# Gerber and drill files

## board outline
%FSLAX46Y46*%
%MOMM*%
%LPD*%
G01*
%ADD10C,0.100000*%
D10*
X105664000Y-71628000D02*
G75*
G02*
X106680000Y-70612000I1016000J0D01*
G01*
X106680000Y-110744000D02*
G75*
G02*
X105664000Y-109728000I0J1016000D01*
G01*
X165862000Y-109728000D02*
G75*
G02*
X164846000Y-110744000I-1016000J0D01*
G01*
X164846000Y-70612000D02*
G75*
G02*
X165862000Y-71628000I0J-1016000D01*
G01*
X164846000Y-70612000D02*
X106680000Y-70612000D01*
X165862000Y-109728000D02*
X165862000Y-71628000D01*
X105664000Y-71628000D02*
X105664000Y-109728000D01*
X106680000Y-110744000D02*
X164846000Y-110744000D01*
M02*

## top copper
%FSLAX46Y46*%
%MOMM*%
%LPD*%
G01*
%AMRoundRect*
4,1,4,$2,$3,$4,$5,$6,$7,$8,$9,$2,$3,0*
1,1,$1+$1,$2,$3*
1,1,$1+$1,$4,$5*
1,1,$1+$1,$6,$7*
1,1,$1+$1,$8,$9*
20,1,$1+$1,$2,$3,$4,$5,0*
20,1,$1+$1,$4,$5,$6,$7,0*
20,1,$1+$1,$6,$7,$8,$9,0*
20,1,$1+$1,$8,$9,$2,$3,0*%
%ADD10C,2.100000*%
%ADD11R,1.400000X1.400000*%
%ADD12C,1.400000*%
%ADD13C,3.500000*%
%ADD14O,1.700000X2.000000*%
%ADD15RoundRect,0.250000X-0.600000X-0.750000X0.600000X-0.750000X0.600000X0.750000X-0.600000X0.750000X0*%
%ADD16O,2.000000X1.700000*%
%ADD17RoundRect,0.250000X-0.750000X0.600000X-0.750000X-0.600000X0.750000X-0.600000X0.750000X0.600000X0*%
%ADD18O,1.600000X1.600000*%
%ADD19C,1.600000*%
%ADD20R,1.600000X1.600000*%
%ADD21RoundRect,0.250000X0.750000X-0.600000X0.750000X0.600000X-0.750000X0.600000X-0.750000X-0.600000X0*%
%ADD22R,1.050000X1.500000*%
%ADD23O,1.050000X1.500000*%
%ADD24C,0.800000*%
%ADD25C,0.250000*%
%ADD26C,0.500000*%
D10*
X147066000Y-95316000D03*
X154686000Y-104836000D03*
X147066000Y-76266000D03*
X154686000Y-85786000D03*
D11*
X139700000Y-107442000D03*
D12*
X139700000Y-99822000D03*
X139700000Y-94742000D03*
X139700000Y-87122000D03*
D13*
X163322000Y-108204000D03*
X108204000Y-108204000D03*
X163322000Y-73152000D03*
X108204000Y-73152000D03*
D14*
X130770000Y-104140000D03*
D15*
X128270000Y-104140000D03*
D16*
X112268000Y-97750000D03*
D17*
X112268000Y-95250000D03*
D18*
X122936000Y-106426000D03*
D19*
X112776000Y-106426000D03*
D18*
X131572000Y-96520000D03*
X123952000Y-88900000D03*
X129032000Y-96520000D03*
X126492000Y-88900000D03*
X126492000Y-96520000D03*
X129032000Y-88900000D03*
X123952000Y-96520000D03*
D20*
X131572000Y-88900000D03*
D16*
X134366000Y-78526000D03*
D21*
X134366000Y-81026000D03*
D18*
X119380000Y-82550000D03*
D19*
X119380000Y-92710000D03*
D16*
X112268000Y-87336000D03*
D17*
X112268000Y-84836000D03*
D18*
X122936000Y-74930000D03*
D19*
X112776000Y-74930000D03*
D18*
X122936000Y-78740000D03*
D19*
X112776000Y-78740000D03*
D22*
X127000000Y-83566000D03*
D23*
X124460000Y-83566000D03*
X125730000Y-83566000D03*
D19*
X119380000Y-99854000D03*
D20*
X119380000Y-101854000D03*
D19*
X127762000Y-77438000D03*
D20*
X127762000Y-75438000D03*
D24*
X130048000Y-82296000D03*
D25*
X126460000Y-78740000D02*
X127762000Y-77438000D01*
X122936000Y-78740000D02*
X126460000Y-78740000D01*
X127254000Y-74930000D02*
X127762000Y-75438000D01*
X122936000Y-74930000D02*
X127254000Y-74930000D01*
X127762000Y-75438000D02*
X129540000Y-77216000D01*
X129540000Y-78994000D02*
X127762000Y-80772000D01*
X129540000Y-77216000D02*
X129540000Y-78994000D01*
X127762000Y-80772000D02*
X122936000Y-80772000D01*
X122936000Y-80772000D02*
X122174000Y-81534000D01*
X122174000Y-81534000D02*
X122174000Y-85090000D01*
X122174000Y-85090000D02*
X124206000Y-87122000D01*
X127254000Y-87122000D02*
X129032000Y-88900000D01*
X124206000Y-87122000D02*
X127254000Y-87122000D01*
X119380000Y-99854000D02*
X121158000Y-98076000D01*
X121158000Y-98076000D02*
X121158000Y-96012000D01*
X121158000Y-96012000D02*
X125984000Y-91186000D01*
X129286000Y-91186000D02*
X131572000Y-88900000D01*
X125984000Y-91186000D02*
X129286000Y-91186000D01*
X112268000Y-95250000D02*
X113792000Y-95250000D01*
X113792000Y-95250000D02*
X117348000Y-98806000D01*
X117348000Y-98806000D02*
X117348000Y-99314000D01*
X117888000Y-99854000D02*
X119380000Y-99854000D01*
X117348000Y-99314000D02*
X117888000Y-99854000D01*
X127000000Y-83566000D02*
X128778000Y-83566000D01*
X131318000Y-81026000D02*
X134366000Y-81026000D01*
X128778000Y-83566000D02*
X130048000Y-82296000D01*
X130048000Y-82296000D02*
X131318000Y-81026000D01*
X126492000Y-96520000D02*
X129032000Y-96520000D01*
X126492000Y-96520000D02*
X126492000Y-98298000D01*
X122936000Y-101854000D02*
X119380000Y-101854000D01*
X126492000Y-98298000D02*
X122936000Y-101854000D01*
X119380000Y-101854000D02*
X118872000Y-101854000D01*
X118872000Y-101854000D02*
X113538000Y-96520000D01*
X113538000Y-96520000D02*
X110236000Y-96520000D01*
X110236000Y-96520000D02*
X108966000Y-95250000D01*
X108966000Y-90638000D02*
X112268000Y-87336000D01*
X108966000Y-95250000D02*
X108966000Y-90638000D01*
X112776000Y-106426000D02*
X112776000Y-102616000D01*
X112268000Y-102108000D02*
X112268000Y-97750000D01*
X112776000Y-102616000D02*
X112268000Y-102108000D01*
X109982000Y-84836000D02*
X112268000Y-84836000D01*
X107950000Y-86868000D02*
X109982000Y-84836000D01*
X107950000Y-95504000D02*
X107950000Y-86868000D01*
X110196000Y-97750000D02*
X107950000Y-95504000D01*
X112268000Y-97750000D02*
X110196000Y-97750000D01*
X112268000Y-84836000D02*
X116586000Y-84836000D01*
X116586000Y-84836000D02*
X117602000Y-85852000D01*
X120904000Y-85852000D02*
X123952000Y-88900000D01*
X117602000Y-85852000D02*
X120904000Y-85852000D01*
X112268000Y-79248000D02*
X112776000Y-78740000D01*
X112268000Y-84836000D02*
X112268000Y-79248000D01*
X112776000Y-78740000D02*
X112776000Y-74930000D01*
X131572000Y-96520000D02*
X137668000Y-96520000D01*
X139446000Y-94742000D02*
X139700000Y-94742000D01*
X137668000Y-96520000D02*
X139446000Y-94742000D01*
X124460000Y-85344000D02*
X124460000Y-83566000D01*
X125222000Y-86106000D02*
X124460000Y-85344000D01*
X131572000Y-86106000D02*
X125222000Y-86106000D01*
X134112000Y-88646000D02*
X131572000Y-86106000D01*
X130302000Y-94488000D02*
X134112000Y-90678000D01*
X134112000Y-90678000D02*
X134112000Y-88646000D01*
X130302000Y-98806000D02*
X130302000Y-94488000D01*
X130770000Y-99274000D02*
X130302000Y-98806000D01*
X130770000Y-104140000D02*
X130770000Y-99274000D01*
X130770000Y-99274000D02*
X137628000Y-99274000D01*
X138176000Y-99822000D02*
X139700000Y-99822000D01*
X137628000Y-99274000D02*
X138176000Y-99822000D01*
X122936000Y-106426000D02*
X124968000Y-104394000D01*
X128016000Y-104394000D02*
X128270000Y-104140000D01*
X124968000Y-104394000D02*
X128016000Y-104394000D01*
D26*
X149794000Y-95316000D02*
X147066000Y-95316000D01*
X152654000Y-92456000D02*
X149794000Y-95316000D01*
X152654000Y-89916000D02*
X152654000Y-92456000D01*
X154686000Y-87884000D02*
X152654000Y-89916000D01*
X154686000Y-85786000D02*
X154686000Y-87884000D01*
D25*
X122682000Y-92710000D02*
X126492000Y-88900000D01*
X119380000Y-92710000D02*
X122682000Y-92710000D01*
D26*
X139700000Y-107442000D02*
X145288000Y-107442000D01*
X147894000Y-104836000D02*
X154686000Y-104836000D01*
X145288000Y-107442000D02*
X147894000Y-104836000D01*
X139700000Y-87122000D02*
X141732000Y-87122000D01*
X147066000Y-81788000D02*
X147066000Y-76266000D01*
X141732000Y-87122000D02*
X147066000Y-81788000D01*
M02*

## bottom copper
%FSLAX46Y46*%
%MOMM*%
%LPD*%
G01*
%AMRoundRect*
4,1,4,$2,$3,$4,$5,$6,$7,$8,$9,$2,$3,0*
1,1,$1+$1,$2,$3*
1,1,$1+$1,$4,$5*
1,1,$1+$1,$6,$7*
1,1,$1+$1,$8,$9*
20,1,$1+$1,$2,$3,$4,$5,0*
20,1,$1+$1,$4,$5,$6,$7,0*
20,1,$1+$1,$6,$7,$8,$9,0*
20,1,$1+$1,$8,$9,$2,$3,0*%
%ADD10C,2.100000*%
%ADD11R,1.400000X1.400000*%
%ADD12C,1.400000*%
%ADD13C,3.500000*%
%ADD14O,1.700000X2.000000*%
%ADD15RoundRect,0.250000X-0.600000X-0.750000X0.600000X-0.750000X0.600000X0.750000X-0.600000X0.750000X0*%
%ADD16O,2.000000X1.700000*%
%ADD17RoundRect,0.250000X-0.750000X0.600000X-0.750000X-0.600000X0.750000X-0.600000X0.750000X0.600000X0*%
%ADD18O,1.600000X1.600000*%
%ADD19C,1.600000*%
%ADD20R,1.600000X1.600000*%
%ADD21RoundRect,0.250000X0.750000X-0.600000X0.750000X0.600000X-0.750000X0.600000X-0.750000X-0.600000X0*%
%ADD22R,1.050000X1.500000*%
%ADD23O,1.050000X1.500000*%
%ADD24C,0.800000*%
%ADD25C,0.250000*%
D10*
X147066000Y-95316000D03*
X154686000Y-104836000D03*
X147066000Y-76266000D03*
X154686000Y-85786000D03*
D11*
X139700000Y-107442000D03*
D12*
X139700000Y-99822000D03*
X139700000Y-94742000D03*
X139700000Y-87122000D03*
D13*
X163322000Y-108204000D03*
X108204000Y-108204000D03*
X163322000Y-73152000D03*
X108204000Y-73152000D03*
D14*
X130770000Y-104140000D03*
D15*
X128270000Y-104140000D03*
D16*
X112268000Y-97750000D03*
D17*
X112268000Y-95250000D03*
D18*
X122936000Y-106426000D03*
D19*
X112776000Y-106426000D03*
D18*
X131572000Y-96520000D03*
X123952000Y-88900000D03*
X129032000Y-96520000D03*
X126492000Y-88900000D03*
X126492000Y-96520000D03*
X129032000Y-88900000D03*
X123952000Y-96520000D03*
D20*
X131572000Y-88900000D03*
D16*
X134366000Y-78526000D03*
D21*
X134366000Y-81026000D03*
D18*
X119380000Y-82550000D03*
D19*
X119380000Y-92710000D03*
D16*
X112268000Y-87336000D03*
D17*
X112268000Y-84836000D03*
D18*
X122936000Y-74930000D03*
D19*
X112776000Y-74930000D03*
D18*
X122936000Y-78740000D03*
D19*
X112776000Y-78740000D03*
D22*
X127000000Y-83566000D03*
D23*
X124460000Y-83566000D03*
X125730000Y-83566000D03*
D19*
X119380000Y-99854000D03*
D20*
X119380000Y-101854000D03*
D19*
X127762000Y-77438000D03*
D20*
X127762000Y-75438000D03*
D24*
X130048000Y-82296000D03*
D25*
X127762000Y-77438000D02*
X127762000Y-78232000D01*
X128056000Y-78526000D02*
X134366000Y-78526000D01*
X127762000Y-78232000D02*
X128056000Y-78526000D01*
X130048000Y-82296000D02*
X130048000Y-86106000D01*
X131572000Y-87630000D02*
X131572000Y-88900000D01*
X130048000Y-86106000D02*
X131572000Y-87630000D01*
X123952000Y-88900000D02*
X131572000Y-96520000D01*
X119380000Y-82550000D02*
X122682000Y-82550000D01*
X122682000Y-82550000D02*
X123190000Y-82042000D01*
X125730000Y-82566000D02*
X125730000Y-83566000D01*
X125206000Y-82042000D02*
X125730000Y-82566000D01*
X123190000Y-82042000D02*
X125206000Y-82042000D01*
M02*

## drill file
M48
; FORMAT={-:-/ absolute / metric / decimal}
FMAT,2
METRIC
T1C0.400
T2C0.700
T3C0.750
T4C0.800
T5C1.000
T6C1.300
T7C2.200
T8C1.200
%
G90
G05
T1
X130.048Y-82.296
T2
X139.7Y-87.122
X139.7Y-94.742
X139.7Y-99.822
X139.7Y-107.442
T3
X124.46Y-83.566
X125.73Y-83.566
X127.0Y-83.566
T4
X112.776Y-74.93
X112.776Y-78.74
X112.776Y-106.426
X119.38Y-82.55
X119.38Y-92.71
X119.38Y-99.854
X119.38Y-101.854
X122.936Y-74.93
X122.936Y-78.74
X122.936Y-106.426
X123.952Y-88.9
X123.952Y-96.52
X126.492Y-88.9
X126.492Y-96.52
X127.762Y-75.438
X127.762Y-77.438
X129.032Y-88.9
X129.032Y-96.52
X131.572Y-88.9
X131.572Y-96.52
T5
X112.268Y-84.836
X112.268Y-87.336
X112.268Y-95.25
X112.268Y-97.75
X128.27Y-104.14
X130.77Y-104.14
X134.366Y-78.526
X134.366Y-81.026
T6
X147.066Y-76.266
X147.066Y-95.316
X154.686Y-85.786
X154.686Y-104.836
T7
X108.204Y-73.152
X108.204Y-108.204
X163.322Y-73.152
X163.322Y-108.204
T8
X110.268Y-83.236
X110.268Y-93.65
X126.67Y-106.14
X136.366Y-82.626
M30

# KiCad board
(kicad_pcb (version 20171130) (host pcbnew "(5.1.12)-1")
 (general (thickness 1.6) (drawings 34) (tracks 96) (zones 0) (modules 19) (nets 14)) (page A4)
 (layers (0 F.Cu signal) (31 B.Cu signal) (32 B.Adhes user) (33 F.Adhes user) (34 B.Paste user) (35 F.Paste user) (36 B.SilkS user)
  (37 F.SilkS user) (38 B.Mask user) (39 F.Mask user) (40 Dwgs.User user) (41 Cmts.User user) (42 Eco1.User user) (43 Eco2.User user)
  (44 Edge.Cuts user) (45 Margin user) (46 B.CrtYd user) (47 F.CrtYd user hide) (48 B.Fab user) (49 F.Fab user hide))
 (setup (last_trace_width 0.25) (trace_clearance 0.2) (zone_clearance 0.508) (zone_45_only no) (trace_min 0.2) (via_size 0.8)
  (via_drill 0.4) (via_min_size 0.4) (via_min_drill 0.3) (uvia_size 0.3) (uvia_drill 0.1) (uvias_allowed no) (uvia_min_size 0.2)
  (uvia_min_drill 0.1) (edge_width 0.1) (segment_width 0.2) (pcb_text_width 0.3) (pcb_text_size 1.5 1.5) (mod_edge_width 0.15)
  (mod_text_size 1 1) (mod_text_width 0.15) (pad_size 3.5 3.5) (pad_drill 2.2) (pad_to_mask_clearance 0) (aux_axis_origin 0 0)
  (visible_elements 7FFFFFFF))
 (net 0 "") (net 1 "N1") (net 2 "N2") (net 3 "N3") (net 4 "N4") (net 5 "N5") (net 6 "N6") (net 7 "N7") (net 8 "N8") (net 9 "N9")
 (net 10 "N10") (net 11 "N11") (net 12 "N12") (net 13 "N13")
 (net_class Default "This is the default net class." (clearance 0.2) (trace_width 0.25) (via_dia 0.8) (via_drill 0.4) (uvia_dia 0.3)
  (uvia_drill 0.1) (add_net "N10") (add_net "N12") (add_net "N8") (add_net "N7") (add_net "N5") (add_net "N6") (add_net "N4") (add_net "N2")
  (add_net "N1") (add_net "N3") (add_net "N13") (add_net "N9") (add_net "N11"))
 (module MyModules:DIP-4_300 (layer F.Cu) (at 150.876 100.076 90)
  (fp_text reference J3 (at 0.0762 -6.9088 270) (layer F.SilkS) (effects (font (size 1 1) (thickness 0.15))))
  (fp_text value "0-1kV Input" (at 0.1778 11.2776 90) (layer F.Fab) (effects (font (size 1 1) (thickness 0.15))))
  (pad 2 thru_hole circle (at 4.76 -3.81 90) (size 2.1 2.1) (drill 1.3) (layers *.Cu *.Mask) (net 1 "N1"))
  (pad 1 thru_hole circle (at -4.76 3.81 90) (size 2.1 2.1) (drill 1.3) (layers *.Cu *.Mask) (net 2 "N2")))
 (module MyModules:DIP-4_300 (layer F.Cu) (at 150.876 81.026 90)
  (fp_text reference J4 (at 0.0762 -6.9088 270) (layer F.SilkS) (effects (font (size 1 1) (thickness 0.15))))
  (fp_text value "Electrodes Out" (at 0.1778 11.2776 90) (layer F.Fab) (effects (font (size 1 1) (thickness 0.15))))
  (pad 2 thru_hole circle (at 4.76 -3.81 90) (size 2.1 2.1) (drill 1.3) (layers *.Cu *.Mask) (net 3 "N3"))
  (pad 1 thru_hole circle (at -4.76 3.81 90) (size 2.1 2.1) (drill 1.3) (layers *.Cu *.Mask) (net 1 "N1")))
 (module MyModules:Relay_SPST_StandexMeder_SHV (layer F.Cu) (at 139.7 107.442 90)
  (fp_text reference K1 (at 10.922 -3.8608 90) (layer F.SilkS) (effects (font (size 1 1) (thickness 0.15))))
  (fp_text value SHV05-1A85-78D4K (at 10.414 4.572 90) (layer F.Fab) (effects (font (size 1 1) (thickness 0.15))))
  (pad 1 thru_hole rect (at 0 0 90) (size 1.4 1.4) (drill 0.7) (layers *.Cu *.Mask) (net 2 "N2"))
  (pad 3 thru_hole circle (at 7.62 0 90) (size 1.4 1.4) (drill 0.7) (layers *.Cu *.Mask) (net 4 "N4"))
  (pad 5 thru_hole circle (at 12.7 0 90) (size 1.4 1.4) (drill 0.7) (layers *.Cu *.Mask) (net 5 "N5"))
  (pad 7 thru_hole circle (at 20.32 0 90) (size 1.4 1.4) (drill 0.7) (layers *.Cu *.Mask) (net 3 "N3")))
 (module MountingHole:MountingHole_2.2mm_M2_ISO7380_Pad (layer F.Cu) (at 163.322 108.204)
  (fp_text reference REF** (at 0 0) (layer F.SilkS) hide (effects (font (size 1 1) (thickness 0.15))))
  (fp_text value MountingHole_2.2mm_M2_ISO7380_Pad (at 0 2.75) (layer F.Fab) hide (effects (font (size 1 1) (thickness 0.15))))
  (pad 1 thru_hole circle (at 0 0) (size 3.5 3.5) (drill 2.2) (layers *.Cu *.Mask)))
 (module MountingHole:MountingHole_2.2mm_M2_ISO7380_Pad (layer F.Cu) (at 108.204 108.204)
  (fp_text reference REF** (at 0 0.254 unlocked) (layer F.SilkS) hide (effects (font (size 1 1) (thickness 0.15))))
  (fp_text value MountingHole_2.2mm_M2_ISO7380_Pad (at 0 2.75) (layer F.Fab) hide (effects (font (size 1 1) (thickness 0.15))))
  (pad 1 thru_hole circle (at 0 0) (size 3.5 3.5) (drill 2.2) (layers *.Cu *.Mask)))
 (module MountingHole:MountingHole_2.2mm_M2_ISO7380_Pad (layer F.Cu) (at 163.322 73.152)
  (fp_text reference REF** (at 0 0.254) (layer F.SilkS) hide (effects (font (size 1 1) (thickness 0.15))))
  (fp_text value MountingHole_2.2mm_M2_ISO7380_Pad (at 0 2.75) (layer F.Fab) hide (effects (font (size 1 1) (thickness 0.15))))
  (pad 1 thru_hole circle (at 0 0) (size 3.5 3.5) (drill 2.2) (layers *.Cu *.Mask)))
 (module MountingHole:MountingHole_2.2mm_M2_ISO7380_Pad (layer F.Cu) (at 108.204 73.152)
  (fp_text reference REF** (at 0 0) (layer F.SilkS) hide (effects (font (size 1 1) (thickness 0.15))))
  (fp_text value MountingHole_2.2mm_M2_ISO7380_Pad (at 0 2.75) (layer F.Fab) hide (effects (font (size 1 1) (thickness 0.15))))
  (pad 1 thru_hole circle (at 0 0) (size 3.5 3.5) (drill 2.2) (layers *.Cu *.Mask)))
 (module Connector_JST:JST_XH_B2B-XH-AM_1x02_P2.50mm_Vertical (layer F.Cu) (at 128.27 104.14)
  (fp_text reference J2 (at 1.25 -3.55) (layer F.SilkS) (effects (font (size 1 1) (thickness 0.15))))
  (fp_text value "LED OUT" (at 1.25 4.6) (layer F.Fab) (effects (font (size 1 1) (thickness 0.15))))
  (pad "" np_thru_hole circle (at -1.6 2) (size 1.2 1.2) (drill 1.2) (layers *.Cu *.Mask))
  (pad 2 thru_hole oval (at 2.5 0) (size 1.7 2) (drill 1) (layers *.Cu *.Mask) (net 4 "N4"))
  (pad 1 thru_hole roundrect (at 0 0) (size 1.7 2) (drill 1) (layers *.Cu *.Mask) (roundrect_rratio 0.147059) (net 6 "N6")))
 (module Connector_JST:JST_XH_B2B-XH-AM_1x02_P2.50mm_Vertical (layer F.Cu) (at 112.268 95.25 270)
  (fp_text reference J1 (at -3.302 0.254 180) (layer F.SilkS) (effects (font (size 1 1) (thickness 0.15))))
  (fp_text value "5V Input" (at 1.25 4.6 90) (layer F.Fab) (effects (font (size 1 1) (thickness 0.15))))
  (pad "" np_thru_hole circle (at -1.6 2 270) (size 1.2 1.2) (drill 1.2) (layers *.Cu *.Mask))
  (pad 2 thru_hole oval (at 2.5 0 270) (size 1.7 2) (drill 1) (layers *.Cu *.Mask) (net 5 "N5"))
  (pad 1 thru_hole roundrect (at 0 0 270) (size 1.7 2) (drill 1) (layers *.Cu *.Mask) (roundrect_rratio 0.147059) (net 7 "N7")))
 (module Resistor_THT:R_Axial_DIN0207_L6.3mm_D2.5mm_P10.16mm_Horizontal (layer F.Cu) (at 112.776 106.426)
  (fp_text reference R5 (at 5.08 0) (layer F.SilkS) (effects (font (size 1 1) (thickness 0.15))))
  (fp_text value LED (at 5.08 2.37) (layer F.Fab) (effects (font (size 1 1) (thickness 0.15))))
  (pad 2 thru_hole oval (at 10.16 0) (size 1.6 1.6) (drill 0.8) (layers *.Cu *.Mask) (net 6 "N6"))
  (pad 1 thru_hole circle (at 0 0) (size 1.6 1.6) (drill 0.8) (layers *.Cu *.Mask) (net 5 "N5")))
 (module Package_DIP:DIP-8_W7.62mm (layer F.Cu) (at 131.572 88.9 270)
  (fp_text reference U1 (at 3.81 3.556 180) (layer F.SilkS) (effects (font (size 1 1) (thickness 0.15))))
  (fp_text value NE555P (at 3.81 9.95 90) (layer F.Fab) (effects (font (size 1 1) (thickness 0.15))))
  (pad 8 thru_hole oval (at 7.62 0 270) (size 1.6 1.6) (drill 0.8) (layers *.Cu *.Mask) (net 5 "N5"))
  (pad 4 thru_hole oval (at 0 7.62 270) (size 1.6 1.6) (drill 0.8) (layers *.Cu *.Mask) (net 5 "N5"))
  (pad 7 thru_hole oval (at 7.62 2.54 270) (size 1.6 1.6) (drill 0.8) (layers *.Cu *.Mask) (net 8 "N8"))
  (pad 3 thru_hole oval (at 0 5.08 270) (size 1.6 1.6) (drill 0.8) (layers *.Cu *.Mask) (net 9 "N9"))
  (pad 6 thru_hole oval (at 7.62 5.08 270) (size 1.6 1.6) (drill 0.8) (layers *.Cu *.Mask) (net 8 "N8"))
  (pad 2 thru_hole oval (at 0 2.54 270) (size 1.6 1.6) (drill 0.8) (layers *.Cu *.Mask) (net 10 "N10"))
  (pad 5 thru_hole oval (at 7.62 7.62 270) (size 1.6 1.6) (drill 0.8) (layers *.Cu *.Mask) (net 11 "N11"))
  (pad 1 thru_hole rect (at 0 0 270) (size 1.6 1.6) (drill 0.8) (layers *.Cu *.Mask) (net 7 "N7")))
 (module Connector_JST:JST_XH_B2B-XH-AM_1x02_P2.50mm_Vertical (layer F.Cu) (at 134.366 81.026 90)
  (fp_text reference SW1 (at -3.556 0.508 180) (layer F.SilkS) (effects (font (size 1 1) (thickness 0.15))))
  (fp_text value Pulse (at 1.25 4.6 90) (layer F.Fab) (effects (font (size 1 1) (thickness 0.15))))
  (pad "" np_thru_hole circle (at -1.6 2 90) (size 1.2 1.2) (drill 1.2) (layers *.Cu *.Mask))
  (pad 2 thru_hole oval (at 2.5 0 90) (size 1.7 2) (drill 1) (layers *.Cu *.Mask) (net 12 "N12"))
  (pad 1 thru_hole roundrect (at 0 0 90) (size 1.7 2) (drill 1) (layers *.Cu *.Mask) (roundrect_rratio 0.147059) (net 7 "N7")))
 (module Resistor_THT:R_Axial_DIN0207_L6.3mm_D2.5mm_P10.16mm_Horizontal (layer F.Cu) (at 119.38 92.71 90)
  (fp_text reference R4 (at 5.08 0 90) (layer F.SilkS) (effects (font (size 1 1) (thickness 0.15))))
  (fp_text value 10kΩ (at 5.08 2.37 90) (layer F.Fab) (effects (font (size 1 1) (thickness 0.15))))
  (pad 2 thru_hole oval (at 10.16 0 90) (size 1.6 1.6) (drill 0.8) (layers *.Cu *.Mask) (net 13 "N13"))
  (pad 1 thru_hole circle (at 0 0 90) (size 1.6 1.6) (drill 0.8) (layers *.Cu *.Mask) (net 9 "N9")))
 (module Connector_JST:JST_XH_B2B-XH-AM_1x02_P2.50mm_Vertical (layer F.Cu) (at 112.268 84.836 270)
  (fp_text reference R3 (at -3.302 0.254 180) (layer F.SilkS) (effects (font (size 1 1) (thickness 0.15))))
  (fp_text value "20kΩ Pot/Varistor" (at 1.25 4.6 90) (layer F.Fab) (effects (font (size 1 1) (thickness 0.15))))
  (pad "" np_thru_hole circle (at -1.6 2 270) (size 1.2 1.2) (drill 1.2) (layers *.Cu *.Mask))
  (pad 2 thru_hole oval (at 2.5 0 270) (size 1.7 2) (drill 1) (layers *.Cu *.Mask) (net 8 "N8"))
  (pad 1 thru_hole roundrect (at 0 0 270) (size 1.7 2) (drill 1) (layers *.Cu *.Mask) (roundrect_rratio 0.147059) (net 5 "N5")))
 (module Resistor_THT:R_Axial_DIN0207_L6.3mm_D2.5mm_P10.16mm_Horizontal (layer F.Cu) (at 112.776 74.93)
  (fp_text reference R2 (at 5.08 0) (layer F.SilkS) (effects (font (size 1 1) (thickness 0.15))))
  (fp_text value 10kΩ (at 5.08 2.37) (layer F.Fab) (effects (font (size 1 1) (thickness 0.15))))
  (pad 2 thru_hole oval (at 10.16 0) (size 1.6 1.6) (drill 0.8) (layers *.Cu *.Mask) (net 10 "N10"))
  (pad 1 thru_hole circle (at 0 0) (size 1.6 1.6) (drill 0.8) (layers *.Cu *.Mask) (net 5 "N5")))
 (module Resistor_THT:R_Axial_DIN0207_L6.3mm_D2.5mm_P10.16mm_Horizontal (layer F.Cu) (at 112.776 78.74)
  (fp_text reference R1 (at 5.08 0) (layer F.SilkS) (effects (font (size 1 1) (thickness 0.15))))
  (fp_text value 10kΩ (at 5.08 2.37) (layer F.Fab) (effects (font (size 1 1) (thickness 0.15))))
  (pad 2 thru_hole oval (at 10.16 0) (size 1.6 1.6) (drill 0.8) (layers *.Cu *.Mask) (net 12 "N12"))
  (pad 1 thru_hole circle (at 0 0) (size 1.6 1.6) (drill 0.8) (layers *.Cu *.Mask) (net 5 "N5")))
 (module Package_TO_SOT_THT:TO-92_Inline (layer F.Cu) (at 127 83.566 180)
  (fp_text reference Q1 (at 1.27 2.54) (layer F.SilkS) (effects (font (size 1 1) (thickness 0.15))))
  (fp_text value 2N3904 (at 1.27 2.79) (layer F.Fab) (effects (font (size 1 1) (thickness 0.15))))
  (pad 1 thru_hole rect (at 0 0 180) (size 1.05 1.5) (drill 0.75) (layers *.Cu *.Mask) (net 7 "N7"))
  (pad 3 thru_hole oval (at 2.54 0 180) (size 1.05 1.5) (drill 0.75) (layers *.Cu *.Mask) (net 4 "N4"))
  (pad 2 thru_hole oval (at 1.27 0 180) (size 1.05 1.5) (drill 0.75) (layers *.Cu *.Mask) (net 13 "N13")))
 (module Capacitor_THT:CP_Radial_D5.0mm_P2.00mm (layer F.Cu) (at 119.38 101.854 90)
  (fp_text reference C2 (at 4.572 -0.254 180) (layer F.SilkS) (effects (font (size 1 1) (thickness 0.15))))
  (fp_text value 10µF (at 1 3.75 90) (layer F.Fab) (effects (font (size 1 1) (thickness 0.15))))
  (pad 2 thru_hole circle (at 2 0 90) (size 1.6 1.6) (drill 0.8) (layers *.Cu *.Mask) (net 7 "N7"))
  (pad 1 thru_hole rect (at 0 0 90) (size 1.6 1.6) (drill 0.8) (layers *.Cu *.Mask) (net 8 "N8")))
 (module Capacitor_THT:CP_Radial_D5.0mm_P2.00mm (layer F.Cu) (at 127.762 75.438 270)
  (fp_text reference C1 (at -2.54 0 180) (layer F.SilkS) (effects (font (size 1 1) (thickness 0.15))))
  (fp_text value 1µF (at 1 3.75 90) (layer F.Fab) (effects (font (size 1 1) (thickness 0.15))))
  (pad 2 thru_hole circle (at 2 0 270) (size 1.6 1.6) (drill 0.8) (layers *.Cu *.Mask) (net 12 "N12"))
  (pad 1 thru_hole rect (at 0 0 270) (size 1.6 1.6) (drill 0.8) (layers *.Cu *.Mask) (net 10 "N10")))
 (gr_arc (start 106.68 71.628) (end 106.68 70.612) (angle -90) (layer Edge.Cuts) (width 0.1))
 (gr_arc (start 106.68 109.728) (end 105.664 109.728) (angle -90) (layer Edge.Cuts) (width 0.1))
 (gr_arc (start 164.846 109.728) (end 164.846 110.744) (angle -90) (layer Edge.Cuts) (width 0.1))
 (gr_arc (start 164.846 71.628) (end 165.862 71.628) (angle -90) (layer Edge.Cuts) (width 0.1))
 (gr_line (start 164.846 70.612) (end 106.68 70.612) (layer Edge.Cuts) (width 0.1))
 (gr_line (start 165.862 109.728) (end 165.862 71.628) (layer Edge.Cuts) (width 0.1))
 (gr_line (start 105.664 71.628) (end 105.664 109.728) (layer Edge.Cuts) (width 0.1))
 (gr_line (start 106.68 110.744) (end 164.846 110.744) (layer Edge.Cuts) (width 0.1))
 (segment (start 126.46 78.74) (end 127.762 77.438) (width 0.25) (layer F.Cu) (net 12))
 (segment (start 122.936 78.74) (end 126.46 78.74) (width 0.25) (layer F.Cu) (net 12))
 (segment (start 127.762 77.438) (end 127.762 78.232) (width 0.25) (layer B.Cu) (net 12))
 (segment (start 128.056 78.526) (end 134.366 78.526) (width 0.25) (layer B.Cu) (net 12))
 (segment (start 127.762 78.232) (end 128.056 78.526) (width 0.25) (layer B.Cu) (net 12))
 (segment (start 127.254 74.93) (end 127.762 75.438) (width 0.25) (layer F.Cu) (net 10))
 (segment (start 122.936 74.93) (end 127.254 74.93) (width 0.25) (layer F.Cu) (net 10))
 (segment (start 127.762 75.438) (end 129.54 77.216) (width 0.25) (layer F.Cu) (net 10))
 (segment (start 129.54 78.994) (end 127.762 80.772) (width 0.25) (layer F.Cu) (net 10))
 (segment (start 129.54 77.216) (end 129.54 78.994) (width 0.25) (layer F.Cu) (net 10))
 (segment (start 127.762 80.772) (end 122.936 80.772) (width 0.25) (layer F.Cu) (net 10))
 (segment (start 122.936 80.772) (end 122.174 81.534) (width 0.25) (layer F.Cu) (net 10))
 (segment (start 122.174 81.534) (end 122.174 85.09) (width 0.25) (layer F.Cu) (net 10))
 (segment (start 122.174 85.09) (end 124.206 87.122) (width 0.25) (layer F.Cu) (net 10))
 (segment (start 127.254 87.122) (end 129.032 88.9) (width 0.25) (layer F.Cu) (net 10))
 (segment (start 124.206 87.122) (end 127.254 87.122) (width 0.25) (layer F.Cu) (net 10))
 (segment (start 119.38 99.854) (end 121.158 98.076) (width 0.25) (layer F.Cu) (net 7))
 (segment (start 121.158 98.076) (end 121.158 96.012) (width 0.25) (layer F.Cu) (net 7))
 (segment (start 121.158 96.012) (end 125.984 91.186) (width 0.25) (layer F.Cu) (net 7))
 (segment (start 129.286 91.186) (end 131.572 88.9) (width 0.25) (layer F.Cu) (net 7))
 (segment (start 125.984 91.186) (end 129.286 91.186) (width 0.25) (layer F.Cu) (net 7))
 (segment (start 112.268 95.25) (end 113.792 95.25) (width 0.25) (layer F.Cu) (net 7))
 (segment (start 113.792 95.25) (end 117.348 98.806) (width 0.25) (layer F.Cu) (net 7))
 (segment (start 117.348 98.806) (end 117.348 99.314) (width 0.25) (layer F.Cu) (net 7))
 (segment (start 117.888 99.854) (end 119.38 99.854) (width 0.25) (layer F.Cu) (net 7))
 (segment (start 117.348 99.314) (end 117.888 99.854) (width 0.25) (layer F.Cu) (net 7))
 (segment (start 127 83.566) (end 128.778 83.566) (width 0.25) (layer F.Cu) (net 7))
 (segment (start 131.318 81.026) (end 134.366 81.026) (width 0.25) (layer F.Cu) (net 7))
 (segment (start 128.778 83.566) (end 130.048 82.296) (width 0.25) (layer F.Cu) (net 7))
 (segment (start 130.048 82.296) (end 131.318 81.026) (width 0.25) (layer F.Cu) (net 7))
 (via (at 130.048 82.296) (size 0.8) (drill 0.4) (layers F.Cu B.Cu) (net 7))
 (segment (start 130.048 82.296) (end 130.048 86.106) (width 0.25) (layer B.Cu) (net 7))
 (segment (start 131.572 87.63) (end 131.572 88.9) (width 0.25) (layer B.Cu) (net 7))
 (segment (start 130.048 86.106) (end 131.572 87.63) (width 0.25) (layer B.Cu) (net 7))
 (segment (start 126.492 96.52) (end 129.032 96.52) (width 0.25) (layer F.Cu) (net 8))
 (segment (start 126.492 96.52) (end 126.492 98.298) (width 0.25) (layer F.Cu) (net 8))
 (segment (start 122.936 101.854) (end 119.38 101.854) (width 0.25) (layer F.Cu) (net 8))
 (segment (start 126.492 98.298) (end 122.936 101.854) (width 0.25) (layer F.Cu) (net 8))
 (segment (start 119.38 101.854) (end 118.872 101.854) (width 0.25) (layer F.Cu) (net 8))
 (segment (start 118.872 101.854) (end 113.538 96.52) (width 0.25) (layer F.Cu) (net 8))
 (segment (start 113.538 96.52) (end 110.236 96.52) (width 0.25) (layer F.Cu) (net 8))
 (segment (start 110.236 96.52) (end 108.966 95.25) (width 0.25) (layer F.Cu) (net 8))
 (segment (start 108.966 90.638) (end 112.268 87.336) (width 0.25) (layer F.Cu) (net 8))
 (segment (start 108.966 95.25) (end 108.966 90.638) (width 0.25) (layer F.Cu) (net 8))
 (segment (start 112.776 106.426) (end 112.776 102.616) (width 0.25) (layer F.Cu) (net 5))
 (segment (start 112.268 102.108) (end 112.268 97.75) (width 0.25) (layer F.Cu) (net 5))
 (segment (start 112.776 102.616) (end 112.268 102.108) (width 0.25) (layer F.Cu) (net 5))
 (segment (start 109.982 84.836) (end 112.268 84.836) (width 0.25) (layer F.Cu) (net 5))
 (segment (start 107.95 86.868) (end 109.982 84.836) (width 0.25) (layer F.Cu) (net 5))
 (segment (start 107.95 95.504) (end 107.95 86.868) (width 0.25) (layer F.Cu) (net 5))
 (segment (start 110.196 97.75) (end 107.95 95.504) (width 0.25) (layer F.Cu) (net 5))
 (segment (start 112.268 97.75) (end 110.196 97.75) (width 0.25) (layer F.Cu) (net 5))
 (segment (start 112.268 84.836) (end 116.586 84.836) (width 0.25) (layer F.Cu) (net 5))
 (segment (start 116.586 84.836) (end 117.602 85.852) (width 0.25) (layer F.Cu) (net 5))
 (segment (start 120.904 85.852) (end 123.952 88.9) (width 0.25) (layer F.Cu) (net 5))
 (segment (start 117.602 85.852) (end 120.904 85.852) (width 0.25) (layer F.Cu) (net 5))
 (segment (start 112.268 79.248) (end 112.776 78.74) (width 0.25) (layer F.Cu) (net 5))
 (segment (start 112.268 84.836) (end 112.268 79.248) (width 0.25) (layer F.Cu) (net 5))
 (segment (start 112.776 78.74) (end 112.776 74.93) (width 0.25) (layer F.Cu) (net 5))
 (segment (start 123.952 88.9) (end 131.572 96.52) (width 0.25) (layer B.Cu) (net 5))
 (segment (start 131.572 96.52) (end 137.668 96.52) (width 0.25) (layer F.Cu) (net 5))
 (segment (start 139.446 94.742) (end 139.7 94.742) (width 0.25) (layer F.Cu) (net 5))
 (segment (start 137.668 96.52) (end 139.446 94.742) (width 0.25) (layer F.Cu) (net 5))
 (segment (start 124.46 85.344) (end 124.46 83.566) (width 0.25) (layer F.Cu) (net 4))
 (segment (start 125.222 86.106) (end 124.46 85.344) (width 0.25) (layer F.Cu) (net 4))
 (segment (start 131.572 86.106) (end 125.222 86.106) (width 0.25) (layer F.Cu) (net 4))
 (segment (start 134.112 88.646) (end 131.572 86.106) (width 0.25) (layer F.Cu) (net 4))
 (segment (start 130.302 94.488) (end 134.112 90.678) (width 0.25) (layer F.Cu) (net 4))
 (segment (start 134.112 90.678) (end 134.112 88.646) (width 0.25) (layer F.Cu) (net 4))
 (segment (start 130.302 98.806) (end 130.302 94.488) (width 0.25) (layer F.Cu) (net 4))
 (segment (start 130.77 99.274) (end 130.302 98.806) (width 0.25) (layer F.Cu) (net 4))
 (segment (start 130.77 104.14) (end 130.77 99.274) (width 0.25) (layer F.Cu) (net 4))
 (segment (start 130.77 99.274) (end 137.628 99.274) (width 0.25) (layer F.Cu) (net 4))
 (segment (start 138.176 99.822) (end 139.7 99.822) (width 0.25) (layer F.Cu) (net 4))
 (segment (start 137.628 99.274) (end 138.176 99.822) (width 0.25) (layer F.Cu) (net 4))
 (segment (start 122.936 106.426) (end 124.968 104.394) (width 0.25) (layer F.Cu) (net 6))
 (segment (start 128.016 104.394) (end 128.27 104.14) (width 0.25) (layer F.Cu) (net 6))
 (segment (start 124.968 104.394) (end 128.016 104.394) (width 0.25) (layer F.Cu) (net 6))
 (segment (start 149.794 95.316) (end 147.066 95.316) (width 0.5) (layer F.Cu) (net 1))
 (segment (start 152.654 92.456) (end 149.794 95.316) (width 0.5) (layer F.Cu) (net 1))
 (segment (start 152.654 89.916) (end 152.654 92.456) (width 0.5) (layer F.Cu) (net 1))
 (segment (start 154.686 87.884) (end 152.654 89.916) (width 0.5) (layer F.Cu) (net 1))
 (segment (start 154.686 85.786) (end 154.686 87.884) (width 0.5) (layer F.Cu) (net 1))
 (segment (start 119.38 82.55) (end 122.682 82.55) (width 0.25) (layer B.Cu) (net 13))
 (segment (start 122.682 82.55) (end 123.19 82.042) (width 0.25) (layer B.Cu) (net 13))
 (segment (start 125.73 82.566) (end 125.73 83.566) (width 0.25) (layer B.Cu) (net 13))
 (segment (start 125.206 82.042) (end 125.73 82.566) (width 0.25) (layer B.Cu) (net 13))
 (segment (start 123.19 82.042) (end 125.206 82.042) (width 0.25) (layer B.Cu) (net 13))
 (segment (start 122.682 92.71) (end 126.492 88.9) (width 0.25) (layer F.Cu) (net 9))
 (segment (start 119.38 92.71) (end 122.682 92.71) (width 0.25) (layer F.Cu) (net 9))
 (segment (start 139.7 107.442) (end 145.288 107.442) (width 0.5) (layer F.Cu) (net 2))
 (segment (start 147.894 104.836) (end 154.686 104.836) (width 0.5) (layer F.Cu) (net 2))
 (segment (start 145.288 107.442) (end 147.894 104.836) (width 0.5) (layer F.Cu) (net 2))
 (segment (start 139.7 87.122) (end 141.732 87.122) (width 0.5) (layer F.Cu) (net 3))
 (segment (start 147.066 81.788) (end 147.066 76.266) (width 0.5) (layer F.Cu) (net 3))
 (segment (start 141.732 87.122) (end 147.066 81.788) (width 0.5) (layer F.Cu) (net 3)))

